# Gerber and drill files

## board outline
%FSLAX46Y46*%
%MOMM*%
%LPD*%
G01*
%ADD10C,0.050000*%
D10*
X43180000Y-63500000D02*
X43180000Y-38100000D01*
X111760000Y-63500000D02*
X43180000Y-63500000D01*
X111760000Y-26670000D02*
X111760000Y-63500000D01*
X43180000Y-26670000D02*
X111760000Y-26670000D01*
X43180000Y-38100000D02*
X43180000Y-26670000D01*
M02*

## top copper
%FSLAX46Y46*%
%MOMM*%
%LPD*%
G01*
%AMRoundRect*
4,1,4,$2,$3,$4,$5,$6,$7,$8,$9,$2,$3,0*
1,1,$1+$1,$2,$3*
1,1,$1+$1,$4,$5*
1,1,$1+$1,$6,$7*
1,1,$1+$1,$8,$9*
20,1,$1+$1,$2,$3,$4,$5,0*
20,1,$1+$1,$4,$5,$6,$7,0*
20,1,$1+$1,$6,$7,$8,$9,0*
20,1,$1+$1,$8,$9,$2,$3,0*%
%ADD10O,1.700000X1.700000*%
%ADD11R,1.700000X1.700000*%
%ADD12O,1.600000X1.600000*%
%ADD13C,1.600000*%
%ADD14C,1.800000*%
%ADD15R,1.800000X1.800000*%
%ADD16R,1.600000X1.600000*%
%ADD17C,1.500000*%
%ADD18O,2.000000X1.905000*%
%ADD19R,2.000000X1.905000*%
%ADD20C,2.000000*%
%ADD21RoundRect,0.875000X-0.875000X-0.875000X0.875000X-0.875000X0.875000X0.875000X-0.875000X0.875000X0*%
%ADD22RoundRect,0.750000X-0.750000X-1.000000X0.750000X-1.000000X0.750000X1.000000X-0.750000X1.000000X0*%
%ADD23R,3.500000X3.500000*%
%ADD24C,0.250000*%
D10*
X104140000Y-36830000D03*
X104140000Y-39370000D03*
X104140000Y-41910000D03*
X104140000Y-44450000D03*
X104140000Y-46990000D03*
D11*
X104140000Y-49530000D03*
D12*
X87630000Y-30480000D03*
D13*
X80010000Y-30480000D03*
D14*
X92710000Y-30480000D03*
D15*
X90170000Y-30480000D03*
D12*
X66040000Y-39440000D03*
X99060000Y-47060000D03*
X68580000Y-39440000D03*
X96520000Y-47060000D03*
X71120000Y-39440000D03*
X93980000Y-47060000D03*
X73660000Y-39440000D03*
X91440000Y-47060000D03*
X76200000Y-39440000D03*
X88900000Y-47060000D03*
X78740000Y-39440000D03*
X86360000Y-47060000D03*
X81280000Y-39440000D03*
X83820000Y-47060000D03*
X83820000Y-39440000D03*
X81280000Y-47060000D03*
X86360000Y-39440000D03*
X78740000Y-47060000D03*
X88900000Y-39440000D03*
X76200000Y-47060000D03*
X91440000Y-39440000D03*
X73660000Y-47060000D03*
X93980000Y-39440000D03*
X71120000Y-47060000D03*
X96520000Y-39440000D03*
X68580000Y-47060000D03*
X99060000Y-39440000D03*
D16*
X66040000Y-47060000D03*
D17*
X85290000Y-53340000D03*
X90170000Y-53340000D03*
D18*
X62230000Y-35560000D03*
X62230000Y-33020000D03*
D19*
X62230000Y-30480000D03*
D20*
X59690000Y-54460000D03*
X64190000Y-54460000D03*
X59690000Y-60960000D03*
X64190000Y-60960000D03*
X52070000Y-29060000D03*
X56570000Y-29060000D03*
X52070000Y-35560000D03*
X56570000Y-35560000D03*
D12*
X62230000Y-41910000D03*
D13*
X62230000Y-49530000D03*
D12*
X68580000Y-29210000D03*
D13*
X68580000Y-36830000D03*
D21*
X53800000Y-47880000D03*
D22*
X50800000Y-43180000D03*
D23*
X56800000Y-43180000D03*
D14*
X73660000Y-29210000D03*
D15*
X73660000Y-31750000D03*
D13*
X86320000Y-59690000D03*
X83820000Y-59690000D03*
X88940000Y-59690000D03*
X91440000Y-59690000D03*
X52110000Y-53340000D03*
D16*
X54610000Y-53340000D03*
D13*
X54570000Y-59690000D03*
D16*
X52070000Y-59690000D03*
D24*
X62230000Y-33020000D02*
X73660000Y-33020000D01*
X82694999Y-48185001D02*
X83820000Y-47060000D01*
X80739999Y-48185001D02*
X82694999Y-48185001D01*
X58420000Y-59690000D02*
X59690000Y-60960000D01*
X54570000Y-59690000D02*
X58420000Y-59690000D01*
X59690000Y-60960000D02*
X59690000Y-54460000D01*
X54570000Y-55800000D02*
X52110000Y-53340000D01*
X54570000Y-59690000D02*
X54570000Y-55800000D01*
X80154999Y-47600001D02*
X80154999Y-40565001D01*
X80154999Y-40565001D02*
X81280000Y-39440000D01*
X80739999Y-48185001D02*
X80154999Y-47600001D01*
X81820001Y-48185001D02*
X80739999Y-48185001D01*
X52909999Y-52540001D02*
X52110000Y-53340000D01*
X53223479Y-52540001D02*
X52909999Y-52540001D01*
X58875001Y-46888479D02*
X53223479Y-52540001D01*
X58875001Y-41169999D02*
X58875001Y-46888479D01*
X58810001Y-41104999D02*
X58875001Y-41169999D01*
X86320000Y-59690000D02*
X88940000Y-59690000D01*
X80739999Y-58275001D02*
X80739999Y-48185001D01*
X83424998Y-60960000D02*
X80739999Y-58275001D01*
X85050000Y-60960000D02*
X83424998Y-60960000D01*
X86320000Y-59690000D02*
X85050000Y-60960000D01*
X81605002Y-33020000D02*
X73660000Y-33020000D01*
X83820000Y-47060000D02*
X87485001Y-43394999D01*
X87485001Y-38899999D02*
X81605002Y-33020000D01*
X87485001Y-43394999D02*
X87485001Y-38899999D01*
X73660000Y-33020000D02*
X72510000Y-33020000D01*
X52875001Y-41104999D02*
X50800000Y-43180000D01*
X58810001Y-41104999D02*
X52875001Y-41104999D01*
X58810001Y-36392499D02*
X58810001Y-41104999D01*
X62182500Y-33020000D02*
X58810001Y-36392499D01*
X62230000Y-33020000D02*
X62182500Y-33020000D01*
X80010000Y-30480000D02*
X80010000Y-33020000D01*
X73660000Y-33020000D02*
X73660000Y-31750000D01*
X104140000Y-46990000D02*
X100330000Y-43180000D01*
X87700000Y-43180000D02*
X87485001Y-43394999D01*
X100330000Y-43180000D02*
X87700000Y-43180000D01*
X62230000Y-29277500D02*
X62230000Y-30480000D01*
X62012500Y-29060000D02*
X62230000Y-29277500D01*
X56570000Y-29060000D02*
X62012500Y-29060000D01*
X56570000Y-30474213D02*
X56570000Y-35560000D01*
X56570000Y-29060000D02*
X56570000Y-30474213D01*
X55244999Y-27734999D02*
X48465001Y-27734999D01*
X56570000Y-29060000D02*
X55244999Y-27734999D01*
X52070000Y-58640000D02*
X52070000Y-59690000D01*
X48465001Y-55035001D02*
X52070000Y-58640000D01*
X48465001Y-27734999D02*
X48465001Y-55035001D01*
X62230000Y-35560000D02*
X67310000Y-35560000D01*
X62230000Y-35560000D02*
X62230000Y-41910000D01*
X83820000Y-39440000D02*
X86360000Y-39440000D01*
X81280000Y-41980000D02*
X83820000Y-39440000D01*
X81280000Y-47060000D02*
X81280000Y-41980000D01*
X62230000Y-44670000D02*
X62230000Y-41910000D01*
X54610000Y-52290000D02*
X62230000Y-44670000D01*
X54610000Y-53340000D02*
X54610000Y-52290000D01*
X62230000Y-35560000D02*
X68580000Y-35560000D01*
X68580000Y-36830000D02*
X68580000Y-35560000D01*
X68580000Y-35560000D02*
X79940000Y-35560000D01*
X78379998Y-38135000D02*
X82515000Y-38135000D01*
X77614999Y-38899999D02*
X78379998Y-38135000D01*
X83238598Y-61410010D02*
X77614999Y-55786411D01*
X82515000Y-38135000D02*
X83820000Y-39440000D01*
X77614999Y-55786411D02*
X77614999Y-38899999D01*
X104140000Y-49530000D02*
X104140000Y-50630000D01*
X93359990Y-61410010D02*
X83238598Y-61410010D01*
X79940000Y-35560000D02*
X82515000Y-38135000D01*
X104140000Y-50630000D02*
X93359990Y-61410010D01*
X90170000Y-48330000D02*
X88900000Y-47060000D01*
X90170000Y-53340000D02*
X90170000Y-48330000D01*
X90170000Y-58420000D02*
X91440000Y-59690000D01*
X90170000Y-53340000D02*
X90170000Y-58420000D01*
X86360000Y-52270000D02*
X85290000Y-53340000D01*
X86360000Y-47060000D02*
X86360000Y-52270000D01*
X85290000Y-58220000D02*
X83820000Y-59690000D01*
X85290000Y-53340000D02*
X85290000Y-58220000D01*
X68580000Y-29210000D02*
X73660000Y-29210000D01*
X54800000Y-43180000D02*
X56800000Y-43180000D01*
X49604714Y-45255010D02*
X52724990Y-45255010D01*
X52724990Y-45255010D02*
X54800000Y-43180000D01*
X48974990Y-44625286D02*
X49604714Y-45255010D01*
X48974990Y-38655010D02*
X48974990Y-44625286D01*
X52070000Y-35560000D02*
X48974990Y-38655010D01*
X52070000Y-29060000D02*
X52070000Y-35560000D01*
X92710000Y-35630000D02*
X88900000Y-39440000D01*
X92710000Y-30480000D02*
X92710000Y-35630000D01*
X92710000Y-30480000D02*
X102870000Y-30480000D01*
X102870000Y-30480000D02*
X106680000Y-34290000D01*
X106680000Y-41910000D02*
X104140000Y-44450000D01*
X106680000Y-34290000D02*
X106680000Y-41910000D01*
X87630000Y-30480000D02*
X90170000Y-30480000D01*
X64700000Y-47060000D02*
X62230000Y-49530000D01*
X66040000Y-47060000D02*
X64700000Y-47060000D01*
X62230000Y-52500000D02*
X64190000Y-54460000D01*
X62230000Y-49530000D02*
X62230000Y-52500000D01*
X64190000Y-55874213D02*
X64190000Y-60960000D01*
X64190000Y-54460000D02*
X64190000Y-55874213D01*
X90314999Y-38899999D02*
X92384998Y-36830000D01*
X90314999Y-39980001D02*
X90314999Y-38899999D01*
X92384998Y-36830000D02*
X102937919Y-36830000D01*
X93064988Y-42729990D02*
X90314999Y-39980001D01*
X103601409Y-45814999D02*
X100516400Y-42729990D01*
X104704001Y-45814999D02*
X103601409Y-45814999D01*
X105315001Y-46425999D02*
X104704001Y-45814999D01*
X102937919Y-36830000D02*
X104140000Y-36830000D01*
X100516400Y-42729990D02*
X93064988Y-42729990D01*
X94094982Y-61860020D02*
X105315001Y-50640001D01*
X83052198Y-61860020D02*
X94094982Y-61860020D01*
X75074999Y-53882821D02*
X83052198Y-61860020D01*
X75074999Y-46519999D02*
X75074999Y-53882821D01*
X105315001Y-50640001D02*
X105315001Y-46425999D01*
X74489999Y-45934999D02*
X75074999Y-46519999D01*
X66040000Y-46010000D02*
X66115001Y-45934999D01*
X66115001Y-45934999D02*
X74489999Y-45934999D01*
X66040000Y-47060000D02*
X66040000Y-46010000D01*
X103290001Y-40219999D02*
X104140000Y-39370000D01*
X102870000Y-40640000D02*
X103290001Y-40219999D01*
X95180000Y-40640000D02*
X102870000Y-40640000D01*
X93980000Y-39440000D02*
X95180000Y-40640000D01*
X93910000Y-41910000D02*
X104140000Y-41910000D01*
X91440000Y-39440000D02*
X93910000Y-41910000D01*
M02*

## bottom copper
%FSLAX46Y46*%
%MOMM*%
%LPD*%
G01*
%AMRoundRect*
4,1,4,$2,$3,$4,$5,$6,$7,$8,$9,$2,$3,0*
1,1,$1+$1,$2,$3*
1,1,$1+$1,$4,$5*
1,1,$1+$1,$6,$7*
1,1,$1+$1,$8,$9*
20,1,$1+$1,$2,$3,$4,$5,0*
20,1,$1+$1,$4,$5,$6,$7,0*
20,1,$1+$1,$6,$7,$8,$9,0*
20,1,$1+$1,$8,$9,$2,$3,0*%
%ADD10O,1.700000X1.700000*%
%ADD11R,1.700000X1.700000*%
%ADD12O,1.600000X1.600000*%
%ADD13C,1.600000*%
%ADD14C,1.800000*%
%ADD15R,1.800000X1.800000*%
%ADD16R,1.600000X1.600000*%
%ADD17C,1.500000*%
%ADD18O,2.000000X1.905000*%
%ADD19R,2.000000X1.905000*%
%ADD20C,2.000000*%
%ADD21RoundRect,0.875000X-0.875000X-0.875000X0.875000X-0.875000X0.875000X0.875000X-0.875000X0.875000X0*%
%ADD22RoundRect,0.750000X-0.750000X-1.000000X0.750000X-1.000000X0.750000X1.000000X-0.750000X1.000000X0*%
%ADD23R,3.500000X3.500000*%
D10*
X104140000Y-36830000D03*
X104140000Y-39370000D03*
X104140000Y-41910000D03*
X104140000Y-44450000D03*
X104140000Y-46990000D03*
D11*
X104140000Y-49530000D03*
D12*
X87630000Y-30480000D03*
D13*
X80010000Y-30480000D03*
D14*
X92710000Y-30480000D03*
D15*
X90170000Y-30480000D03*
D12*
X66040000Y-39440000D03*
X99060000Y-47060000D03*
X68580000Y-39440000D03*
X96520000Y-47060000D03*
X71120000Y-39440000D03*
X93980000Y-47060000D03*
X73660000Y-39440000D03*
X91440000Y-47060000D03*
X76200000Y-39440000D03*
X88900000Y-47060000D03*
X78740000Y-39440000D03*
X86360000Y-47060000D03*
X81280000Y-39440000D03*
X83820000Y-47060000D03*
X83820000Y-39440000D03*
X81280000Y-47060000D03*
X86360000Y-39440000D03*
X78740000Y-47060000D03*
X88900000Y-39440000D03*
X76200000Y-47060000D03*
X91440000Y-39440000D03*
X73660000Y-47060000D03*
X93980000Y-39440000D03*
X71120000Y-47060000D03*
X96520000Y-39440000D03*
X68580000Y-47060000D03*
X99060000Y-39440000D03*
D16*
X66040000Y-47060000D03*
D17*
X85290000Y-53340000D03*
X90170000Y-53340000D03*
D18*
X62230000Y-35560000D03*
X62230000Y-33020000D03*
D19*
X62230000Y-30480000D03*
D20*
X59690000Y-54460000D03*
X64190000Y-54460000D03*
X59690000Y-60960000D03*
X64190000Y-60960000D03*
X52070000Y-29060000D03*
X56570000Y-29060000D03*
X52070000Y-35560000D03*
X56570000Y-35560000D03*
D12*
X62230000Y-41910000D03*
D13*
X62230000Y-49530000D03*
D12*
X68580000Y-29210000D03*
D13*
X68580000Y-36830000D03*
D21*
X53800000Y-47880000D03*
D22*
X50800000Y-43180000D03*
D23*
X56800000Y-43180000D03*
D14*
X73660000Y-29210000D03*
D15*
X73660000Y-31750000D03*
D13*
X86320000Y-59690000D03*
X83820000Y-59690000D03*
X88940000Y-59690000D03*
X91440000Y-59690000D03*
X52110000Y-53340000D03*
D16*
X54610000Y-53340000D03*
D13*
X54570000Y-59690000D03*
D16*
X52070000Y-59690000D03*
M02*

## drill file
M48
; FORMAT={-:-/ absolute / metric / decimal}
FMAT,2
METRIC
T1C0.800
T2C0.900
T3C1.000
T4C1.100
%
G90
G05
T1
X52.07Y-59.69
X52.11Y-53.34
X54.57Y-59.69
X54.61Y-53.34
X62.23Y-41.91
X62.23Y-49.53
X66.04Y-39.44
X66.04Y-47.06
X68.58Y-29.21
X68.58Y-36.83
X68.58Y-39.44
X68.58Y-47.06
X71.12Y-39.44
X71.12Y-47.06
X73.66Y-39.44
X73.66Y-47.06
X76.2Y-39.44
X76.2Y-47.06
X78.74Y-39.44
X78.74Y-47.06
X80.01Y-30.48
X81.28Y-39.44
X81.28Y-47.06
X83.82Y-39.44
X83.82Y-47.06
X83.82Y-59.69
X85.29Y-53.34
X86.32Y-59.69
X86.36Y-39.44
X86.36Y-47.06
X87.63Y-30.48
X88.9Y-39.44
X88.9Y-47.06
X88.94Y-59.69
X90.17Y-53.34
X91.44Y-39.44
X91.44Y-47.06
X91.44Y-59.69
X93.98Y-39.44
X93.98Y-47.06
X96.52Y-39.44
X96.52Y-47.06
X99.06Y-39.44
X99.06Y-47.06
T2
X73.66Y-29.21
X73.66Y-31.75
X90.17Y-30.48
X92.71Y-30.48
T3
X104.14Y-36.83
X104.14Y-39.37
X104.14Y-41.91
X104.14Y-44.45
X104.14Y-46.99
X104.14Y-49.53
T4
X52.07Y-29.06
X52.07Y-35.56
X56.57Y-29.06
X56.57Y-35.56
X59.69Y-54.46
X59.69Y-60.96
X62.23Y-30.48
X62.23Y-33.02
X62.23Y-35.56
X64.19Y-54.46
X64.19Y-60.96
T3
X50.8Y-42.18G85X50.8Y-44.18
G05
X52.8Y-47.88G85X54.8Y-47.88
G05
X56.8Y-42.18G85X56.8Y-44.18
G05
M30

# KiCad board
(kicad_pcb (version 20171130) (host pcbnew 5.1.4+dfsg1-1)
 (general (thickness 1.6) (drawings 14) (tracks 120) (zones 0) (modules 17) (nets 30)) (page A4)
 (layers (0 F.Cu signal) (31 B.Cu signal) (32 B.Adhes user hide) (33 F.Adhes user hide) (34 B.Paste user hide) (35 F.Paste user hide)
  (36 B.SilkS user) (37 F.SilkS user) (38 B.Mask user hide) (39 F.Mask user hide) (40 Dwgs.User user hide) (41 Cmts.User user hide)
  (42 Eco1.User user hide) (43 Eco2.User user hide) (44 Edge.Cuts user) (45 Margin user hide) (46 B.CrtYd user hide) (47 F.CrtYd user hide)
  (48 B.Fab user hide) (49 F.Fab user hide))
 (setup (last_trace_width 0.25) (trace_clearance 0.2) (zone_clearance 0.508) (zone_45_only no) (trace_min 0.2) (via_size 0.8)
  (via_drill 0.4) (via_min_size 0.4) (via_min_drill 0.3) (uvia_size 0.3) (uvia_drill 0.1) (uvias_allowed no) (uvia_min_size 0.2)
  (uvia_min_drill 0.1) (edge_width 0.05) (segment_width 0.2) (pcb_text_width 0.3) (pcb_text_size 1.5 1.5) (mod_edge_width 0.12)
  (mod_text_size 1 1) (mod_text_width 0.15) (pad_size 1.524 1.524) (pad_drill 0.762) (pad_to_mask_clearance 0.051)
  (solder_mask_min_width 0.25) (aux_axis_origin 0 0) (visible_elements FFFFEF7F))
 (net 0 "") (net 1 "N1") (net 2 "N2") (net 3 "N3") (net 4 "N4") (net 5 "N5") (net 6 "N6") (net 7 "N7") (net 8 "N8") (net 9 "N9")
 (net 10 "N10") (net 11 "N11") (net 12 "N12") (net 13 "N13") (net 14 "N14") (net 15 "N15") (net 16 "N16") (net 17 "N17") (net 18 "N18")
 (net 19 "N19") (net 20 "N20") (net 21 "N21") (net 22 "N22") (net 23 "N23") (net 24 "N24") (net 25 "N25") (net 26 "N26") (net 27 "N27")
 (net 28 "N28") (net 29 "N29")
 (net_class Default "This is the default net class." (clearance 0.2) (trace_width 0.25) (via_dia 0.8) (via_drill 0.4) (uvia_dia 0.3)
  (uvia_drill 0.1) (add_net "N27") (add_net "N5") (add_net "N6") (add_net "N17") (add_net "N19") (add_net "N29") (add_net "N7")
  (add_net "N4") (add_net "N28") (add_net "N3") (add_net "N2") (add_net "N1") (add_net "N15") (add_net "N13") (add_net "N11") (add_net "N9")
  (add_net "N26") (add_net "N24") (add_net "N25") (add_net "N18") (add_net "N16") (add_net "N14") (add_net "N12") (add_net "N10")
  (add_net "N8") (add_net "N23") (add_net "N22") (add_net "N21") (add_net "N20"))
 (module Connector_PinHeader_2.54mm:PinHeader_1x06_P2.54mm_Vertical (layer F.Cu) (at 104.14 49.53 180)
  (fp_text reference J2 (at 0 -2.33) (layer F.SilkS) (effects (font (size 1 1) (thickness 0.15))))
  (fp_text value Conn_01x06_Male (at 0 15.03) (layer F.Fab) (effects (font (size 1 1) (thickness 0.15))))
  (pad 6 thru_hole oval (at 0 12.7 180) (size 1.7 1.7) (drill 1) (layers *.Cu *.Mask) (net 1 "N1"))
  (pad 5 thru_hole oval (at 0 10.16 180) (size 1.7 1.7) (drill 1) (layers *.Cu *.Mask) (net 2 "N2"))
  (pad 4 thru_hole oval (at 0 7.62 180) (size 1.7 1.7) (drill 1) (layers *.Cu *.Mask) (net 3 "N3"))
  (pad 3 thru_hole oval (at 0 5.08 180) (size 1.7 1.7) (drill 1) (layers *.Cu *.Mask) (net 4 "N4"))
  (pad 2 thru_hole oval (at 0 2.54 180) (size 1.7 1.7) (drill 1) (layers *.Cu *.Mask) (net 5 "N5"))
  (pad 1 thru_hole rect (at 0 0 180) (size 1.7 1.7) (drill 1) (layers *.Cu *.Mask) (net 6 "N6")))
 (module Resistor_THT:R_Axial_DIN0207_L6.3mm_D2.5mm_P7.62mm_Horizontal (layer F.Cu) (at 80.01 30.48)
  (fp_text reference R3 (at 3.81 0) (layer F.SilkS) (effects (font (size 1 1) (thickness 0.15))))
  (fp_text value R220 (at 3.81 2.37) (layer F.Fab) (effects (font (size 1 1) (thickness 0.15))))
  (pad 2 thru_hole oval (at 7.62 0) (size 1.6 1.6) (drill 0.8) (layers *.Cu *.Mask) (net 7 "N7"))
  (pad 1 thru_hole circle (at 0 0) (size 1.6 1.6) (drill 0.8) (layers *.Cu *.Mask) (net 5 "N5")))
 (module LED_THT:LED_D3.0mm (layer F.Cu) (at 90.17 30.48)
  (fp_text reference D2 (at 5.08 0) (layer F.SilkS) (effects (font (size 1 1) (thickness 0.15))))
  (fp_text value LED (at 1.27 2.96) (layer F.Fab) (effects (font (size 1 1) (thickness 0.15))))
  (pad 2 thru_hole circle (at 2.54 0) (size 1.8 1.8) (drill 0.9) (layers *.Cu *.Mask) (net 4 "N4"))
  (pad 1 thru_hole rect (at 0 0) (size 1.8 1.8) (drill 0.9) (layers *.Cu *.Mask) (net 7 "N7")))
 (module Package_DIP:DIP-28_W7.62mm (layer F.Cu) (at 66.04 47.06 90)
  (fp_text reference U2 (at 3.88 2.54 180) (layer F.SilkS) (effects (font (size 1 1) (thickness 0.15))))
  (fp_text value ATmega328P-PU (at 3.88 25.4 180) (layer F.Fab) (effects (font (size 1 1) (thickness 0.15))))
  (pad 28 thru_hole oval (at 7.62 0 90) (size 1.6 1.6) (drill 0.8) (layers *.Cu *.Mask) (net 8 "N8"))
  (pad 14 thru_hole oval (at 0 33.02 90) (size 1.6 1.6) (drill 0.8) (layers *.Cu *.Mask) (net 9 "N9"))
  (pad 27 thru_hole oval (at 7.62 2.54 90) (size 1.6 1.6) (drill 0.8) (layers *.Cu *.Mask) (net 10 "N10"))
  (pad 13 thru_hole oval (at 0 30.48 90) (size 1.6 1.6) (drill 0.8) (layers *.Cu *.Mask) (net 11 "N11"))
  (pad 26 thru_hole oval (at 7.62 5.08 90) (size 1.6 1.6) (drill 0.8) (layers *.Cu *.Mask) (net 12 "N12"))
  (pad 12 thru_hole oval (at 0 27.94 90) (size 1.6 1.6) (drill 0.8) (layers *.Cu *.Mask) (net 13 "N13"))
  (pad 25 thru_hole oval (at 7.62 7.62 90) (size 1.6 1.6) (drill 0.8) (layers *.Cu *.Mask) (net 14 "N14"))
  (pad 11 thru_hole oval (at 0 25.4 90) (size 1.6 1.6) (drill 0.8) (layers *.Cu *.Mask) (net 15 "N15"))
  (pad 24 thru_hole oval (at 7.62 10.16 90) (size 1.6 1.6) (drill 0.8) (layers *.Cu *.Mask) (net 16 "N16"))
  (pad 10 thru_hole oval (at 0 22.86 90) (size 1.6 1.6) (drill 0.8) (layers *.Cu *.Mask) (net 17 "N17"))
  (pad 23 thru_hole oval (at 7.62 12.7 90) (size 1.6 1.6) (drill 0.8) (layers *.Cu *.Mask) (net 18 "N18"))
  (pad 9 thru_hole oval (at 0 20.32 90) (size 1.6 1.6) (drill 0.8) (layers *.Cu *.Mask) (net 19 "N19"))
  (pad 22 thru_hole oval (at 7.62 15.24 90) (size 1.6 1.6) (drill 0.8) (layers *.Cu *.Mask) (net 5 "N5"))
  (pad 8 thru_hole oval (at 0 17.78 90) (size 1.6 1.6) (drill 0.8) (layers *.Cu *.Mask) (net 5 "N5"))
  (pad 21 thru_hole oval (at 7.62 17.78 90) (size 1.6 1.6) (drill 0.8) (layers *.Cu *.Mask) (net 6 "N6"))
  (pad 7 thru_hole oval (at 0 15.24 90) (size 1.6 1.6) (drill 0.8) (layers *.Cu *.Mask) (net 6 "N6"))
  (pad 20 thru_hole oval (at 7.62 20.32 90) (size 1.6 1.6) (drill 0.8) (layers *.Cu *.Mask) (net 6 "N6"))
  (pad 6 thru_hole oval (at 0 12.7 90) (size 1.6 1.6) (drill 0.8) (layers *.Cu *.Mask) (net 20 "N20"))
  (pad 19 thru_hole oval (at 7.62 22.86 90) (size 1.6 1.6) (drill 0.8) (layers *.Cu *.Mask) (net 4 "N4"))
  (pad 5 thru_hole oval (at 0 10.16 90) (size 1.6 1.6) (drill 0.8) (layers *.Cu *.Mask) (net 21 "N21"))
  (pad 18 thru_hole oval (at 7.62 25.4 90) (size 1.6 1.6) (drill 0.8) (layers *.Cu *.Mask) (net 3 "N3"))
  (pad 4 thru_hole oval (at 0 7.62 90) (size 1.6 1.6) (drill 0.8) (layers *.Cu *.Mask) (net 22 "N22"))
  (pad 17 thru_hole oval (at 7.62 27.94 90) (size 1.6 1.6) (drill 0.8) (layers *.Cu *.Mask) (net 2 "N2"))
  (pad 3 thru_hole oval (at 0 5.08 90) (size 1.6 1.6) (drill 0.8) (layers *.Cu *.Mask) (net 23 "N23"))
  (pad 16 thru_hole oval (at 7.62 30.48 90) (size 1.6 1.6) (drill 0.8) (layers *.Cu *.Mask) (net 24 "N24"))
  (pad 2 thru_hole oval (at 0 2.54 90) (size 1.6 1.6) (drill 0.8) (layers *.Cu *.Mask) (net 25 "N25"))
  (pad 15 thru_hole oval (at 7.62 33.02 90) (size 1.6 1.6) (drill 0.8) (layers *.Cu *.Mask) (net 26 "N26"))
  (pad 1 thru_hole rect (at 0 0 90) (size 1.6 1.6) (drill 0.8) (layers *.Cu *.Mask) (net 1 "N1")))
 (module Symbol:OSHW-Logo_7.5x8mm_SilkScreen (layer F.Cu) (at 73.66 55.88)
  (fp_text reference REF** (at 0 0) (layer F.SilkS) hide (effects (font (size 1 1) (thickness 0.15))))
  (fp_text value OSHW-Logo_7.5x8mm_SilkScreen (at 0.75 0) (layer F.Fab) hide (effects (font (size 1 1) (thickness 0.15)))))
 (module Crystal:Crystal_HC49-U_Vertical (layer F.Cu) (at 90.17 53.34 180)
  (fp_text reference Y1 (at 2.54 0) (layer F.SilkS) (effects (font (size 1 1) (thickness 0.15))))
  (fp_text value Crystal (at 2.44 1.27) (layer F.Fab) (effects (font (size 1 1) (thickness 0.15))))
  (pad 2 thru_hole circle (at 4.88 0 180) (size 1.5 1.5) (drill 0.8) (layers *.Cu *.Mask) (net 19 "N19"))
  (pad 1 thru_hole circle (at 0 0 180) (size 1.5 1.5) (drill 0.8) (layers *.Cu *.Mask) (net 17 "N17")))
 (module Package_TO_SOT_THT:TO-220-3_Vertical (layer F.Cu) (at 62.23 30.48 270)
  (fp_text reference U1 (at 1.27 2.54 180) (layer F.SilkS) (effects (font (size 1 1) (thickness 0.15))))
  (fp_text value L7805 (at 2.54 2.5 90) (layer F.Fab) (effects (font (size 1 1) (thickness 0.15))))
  (pad 3 thru_hole oval (at 5.08 0 270) (size 1.905 2) (drill 1.1) (layers *.Cu *.Mask) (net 6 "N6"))
  (pad 2 thru_hole oval (at 2.54 0 270) (size 1.905 2) (drill 1.1) (layers *.Cu *.Mask) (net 5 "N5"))
  (pad 1 thru_hole rect (at 0 0 270) (size 1.905 2) (drill 1.1) (layers *.Cu *.Mask) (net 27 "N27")))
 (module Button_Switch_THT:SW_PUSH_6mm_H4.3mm (layer F.Cu) (at 59.69 60.96 90)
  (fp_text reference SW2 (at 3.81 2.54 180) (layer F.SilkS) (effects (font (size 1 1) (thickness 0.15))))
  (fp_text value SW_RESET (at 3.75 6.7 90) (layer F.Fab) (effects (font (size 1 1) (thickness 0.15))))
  (pad 1 thru_hole circle (at 6.5 0 180) (size 2 2) (drill 1.1) (layers *.Cu *.Mask) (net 5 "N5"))
  (pad 2 thru_hole circle (at 6.5 4.5 180) (size 2 2) (drill 1.1) (layers *.Cu *.Mask) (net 1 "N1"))
  (pad 1 thru_hole circle (at 0 0 180) (size 2 2) (drill 1.1) (layers *.Cu *.Mask) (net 5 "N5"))
  (pad 2 thru_hole circle (at 0 4.5 180) (size 2 2) (drill 1.1) (layers *.Cu *.Mask) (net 1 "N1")))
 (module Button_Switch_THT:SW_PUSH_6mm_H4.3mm (layer F.Cu) (at 52.07 35.56 90)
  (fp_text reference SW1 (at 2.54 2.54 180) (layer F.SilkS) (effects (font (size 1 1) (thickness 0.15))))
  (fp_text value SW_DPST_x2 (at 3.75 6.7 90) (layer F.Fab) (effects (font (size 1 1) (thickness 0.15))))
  (pad 1 thru_hole circle (at 6.5 0 180) (size 2 2) (drill 1.1) (layers *.Cu *.Mask) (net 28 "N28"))
  (pad 2 thru_hole circle (at 6.5 4.5 180) (size 2 2) (drill 1.1) (layers *.Cu *.Mask) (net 27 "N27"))
  (pad 1 thru_hole circle (at 0 0 180) (size 2 2) (drill 1.1) (layers *.Cu *.Mask) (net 28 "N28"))
  (pad 2 thru_hole circle (at 0 4.5 180) (size 2 2) (drill 1.1) (layers *.Cu *.Mask) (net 27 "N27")))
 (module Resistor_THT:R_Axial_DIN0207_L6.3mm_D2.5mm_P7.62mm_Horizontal (layer F.Cu) (at 62.23 49.53 90)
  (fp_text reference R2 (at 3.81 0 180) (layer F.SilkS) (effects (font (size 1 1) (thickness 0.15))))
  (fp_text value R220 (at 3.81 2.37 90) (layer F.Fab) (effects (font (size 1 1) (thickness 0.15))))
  (pad 2 thru_hole oval (at 7.62 0 90) (size 1.6 1.6) (drill 0.8) (layers *.Cu *.Mask) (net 6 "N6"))
  (pad 1 thru_hole circle (at 0 0 90) (size 1.6 1.6) (drill 0.8) (layers *.Cu *.Mask) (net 1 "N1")))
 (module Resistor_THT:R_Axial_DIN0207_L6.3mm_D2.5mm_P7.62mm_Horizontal (layer F.Cu) (at 68.58 36.83 90)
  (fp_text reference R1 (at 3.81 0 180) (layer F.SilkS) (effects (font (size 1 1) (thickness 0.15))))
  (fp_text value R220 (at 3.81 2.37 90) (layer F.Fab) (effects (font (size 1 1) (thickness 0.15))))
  (pad 2 thru_hole oval (at 7.62 0 90) (size 1.6 1.6) (drill 0.8) (layers *.Cu *.Mask) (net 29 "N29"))
  (pad 1 thru_hole circle (at 0 0 90) (size 1.6 1.6) (drill 0.8) (layers *.Cu *.Mask) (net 6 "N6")))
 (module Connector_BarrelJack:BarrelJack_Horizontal (layer F.Cu) (at 56.8 43.18)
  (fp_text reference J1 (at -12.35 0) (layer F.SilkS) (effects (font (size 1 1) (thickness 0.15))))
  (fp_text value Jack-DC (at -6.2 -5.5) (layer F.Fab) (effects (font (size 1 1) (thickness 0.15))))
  (pad 3 thru_hole roundrect (at -3 4.7) (size 3.5 3.5) (drill oval 3 1) (layers *.Cu *.Mask) (roundrect_rratio 0.25))
  (pad 2 thru_hole roundrect (at -6 0) (size 3 3.5) (drill oval 1 3) (layers *.Cu *.Mask) (roundrect_rratio 0.25) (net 5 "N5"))
  (pad 1 thru_hole rect (at 0 0) (size 3.5 3.5) (drill oval 1 3) (layers *.Cu *.Mask) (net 28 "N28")))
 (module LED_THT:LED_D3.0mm (layer F.Cu) (at 73.66 31.75 90)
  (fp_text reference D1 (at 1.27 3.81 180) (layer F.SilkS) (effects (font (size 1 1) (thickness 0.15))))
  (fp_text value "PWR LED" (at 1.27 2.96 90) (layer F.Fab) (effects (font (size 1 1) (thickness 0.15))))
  (pad 2 thru_hole circle (at 2.54 0 90) (size 1.8 1.8) (drill 0.9) (layers *.Cu *.Mask) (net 29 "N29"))
  (pad 1 thru_hole rect (at 0 0 90) (size 1.8 1.8) (drill 0.9) (layers *.Cu *.Mask) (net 5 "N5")))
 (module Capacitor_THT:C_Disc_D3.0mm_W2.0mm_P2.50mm (layer F.Cu) (at 83.82 59.69)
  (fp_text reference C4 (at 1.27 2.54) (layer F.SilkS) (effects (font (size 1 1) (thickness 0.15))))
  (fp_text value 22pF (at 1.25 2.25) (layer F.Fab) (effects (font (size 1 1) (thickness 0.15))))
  (pad 2 thru_hole circle (at 2.5 0) (size 1.6 1.6) (drill 0.8) (layers *.Cu *.Mask) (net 5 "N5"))
  (pad 1 thru_hole circle (at 0 0) (size 1.6 1.6) (drill 0.8) (layers *.Cu *.Mask) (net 19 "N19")))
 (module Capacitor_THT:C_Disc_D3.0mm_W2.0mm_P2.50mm (layer F.Cu) (at 91.44 59.69 180)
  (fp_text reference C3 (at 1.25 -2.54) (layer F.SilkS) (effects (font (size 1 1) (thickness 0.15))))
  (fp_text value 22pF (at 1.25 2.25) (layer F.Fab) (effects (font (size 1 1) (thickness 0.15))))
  (pad 2 thru_hole circle (at 2.5 0 180) (size 1.6 1.6) (drill 0.8) (layers *.Cu *.Mask) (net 5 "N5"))
  (pad 1 thru_hole circle (at 0 0 180) (size 1.6 1.6) (drill 0.8) (layers *.Cu *.Mask) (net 17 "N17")))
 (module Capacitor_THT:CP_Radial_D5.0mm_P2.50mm (layer F.Cu) (at 54.61 53.34 180)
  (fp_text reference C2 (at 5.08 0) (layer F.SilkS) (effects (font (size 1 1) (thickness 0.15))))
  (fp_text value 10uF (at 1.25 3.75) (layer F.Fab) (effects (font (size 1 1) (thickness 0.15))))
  (pad 2 thru_hole circle (at 2.5 0 180) (size 1.6 1.6) (drill 0.8) (layers *.Cu *.Mask) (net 5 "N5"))
  (pad 1 thru_hole rect (at 0 0 180) (size 1.6 1.6) (drill 0.8) (layers *.Cu *.Mask) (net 6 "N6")))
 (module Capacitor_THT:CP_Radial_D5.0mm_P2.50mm (layer F.Cu) (at 52.07 59.69)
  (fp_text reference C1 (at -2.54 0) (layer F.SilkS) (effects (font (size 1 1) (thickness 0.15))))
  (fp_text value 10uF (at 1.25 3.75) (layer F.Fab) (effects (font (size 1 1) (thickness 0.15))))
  (pad 2 thru_hole circle (at 2.5 0) (size 1.6 1.6) (drill 0.8) (layers *.Cu *.Mask) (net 5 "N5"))
  (pad 1 thru_hole rect (at 0 0) (size 1.6 1.6) (drill 0.8) (layers *.Cu *.Mask) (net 27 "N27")))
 (gr_line (start 43.18 63.5) (end 43.18 38.1) (layer Edge.Cuts) (width 0.05))
 (gr_line (start 111.76 63.5) (end 43.18 63.5) (layer Edge.Cuts) (width 0.05))
 (gr_line (start 111.76 26.67) (end 111.76 63.5) (layer Edge.Cuts) (width 0.05))
 (gr_line (start 43.18 26.67) (end 111.76 26.67) (layer Edge.Cuts) (width 0.05))
 (gr_line (start 43.18 38.1) (end 43.18 26.67) (layer Edge.Cuts) (width 0.05))
 (segment (start 62.23 33.02) (end 73.66 33.02) (width 0.25) (layer F.Cu) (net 5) (status 30))
 (segment (start 82.694999 48.185001) (end 83.82 47.06) (width 0.25) (layer F.Cu) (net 5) (status 20))
 (segment (start 80.739999 48.185001) (end 82.694999 48.185001) (width 0.25) (layer F.Cu) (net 5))
 (segment (start 58.42 59.69) (end 59.69 60.96) (width 0.25) (layer F.Cu) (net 5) (status 20))
 (segment (start 54.57 59.69) (end 58.42 59.69) (width 0.25) (layer F.Cu) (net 5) (status 10))
 (segment (start 59.69 60.96) (end 59.69 54.46) (width 0.25) (layer F.Cu) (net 5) (status 30))
 (segment (start 54.57 55.8) (end 52.11 53.34) (width 0.25) (layer F.Cu) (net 5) (status 20))
 (segment (start 54.57 59.69) (end 54.57 55.8) (width 0.25) (layer F.Cu) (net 5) (status 10))
 (segment (start 80.154999 47.600001) (end 80.154999 40.565001) (width 0.25) (layer F.Cu) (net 5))
 (segment (start 80.154999 40.565001) (end 81.28 39.44) (width 0.25) (layer F.Cu) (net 5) (status 20))
 (segment (start 80.739999 48.185001) (end 80.154999 47.600001) (width 0.25) (layer F.Cu) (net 5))
 (segment (start 81.820001 48.185001) (end 80.739999 48.185001) (width 0.25) (layer F.Cu) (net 5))
 (segment (start 52.909999 52.540001) (end 52.11 53.34) (width 0.25) (layer F.Cu) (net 5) (status 20))
 (segment (start 53.223479 52.540001) (end 52.909999 52.540001) (width 0.25) (layer F.Cu) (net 5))
 (segment (start 58.875001 46.888479) (end 53.223479 52.540001) (width 0.25) (layer F.Cu) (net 5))
 (segment (start 58.875001 41.169999) (end 58.875001 46.888479) (width 0.25) (layer F.Cu) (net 5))
 (segment (start 58.810001 41.104999) (end 58.875001 41.169999) (width 0.25) (layer F.Cu) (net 5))
 (segment (start 86.32 59.69) (end 88.94 59.69) (width 0.25) (layer F.Cu) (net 5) (status 30))
 (segment (start 80.739999 58.275001) (end 80.739999 48.185001) (width 0.25) (layer F.Cu) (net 5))
 (segment (start 83.424998 60.96) (end 80.739999 58.275001) (width 0.25) (layer F.Cu) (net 5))
 (segment (start 85.05 60.96) (end 83.424998 60.96) (width 0.25) (layer F.Cu) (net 5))
 (segment (start 86.32 59.69) (end 85.05 60.96) (width 0.25) (layer F.Cu) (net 5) (status 10))
 (segment (start 81.605002 33.02) (end 73.66 33.02) (width 0.25) (layer F.Cu) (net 5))
 (segment (start 83.82 47.06) (end 87.485001 43.394999) (width 0.25) (layer F.Cu) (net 5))
 (segment (start 87.485001 38.899999) (end 81.605002 33.02) (width 0.25) (layer F.Cu) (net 5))
 (segment (start 87.485001 43.394999) (end 87.485001 38.899999) (width 0.25) (layer F.Cu) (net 5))
 (segment (start 73.66 33.02) (end 72.51 33.02) (width 0.25) (layer F.Cu) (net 5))
 (segment (start 52.875001 41.104999) (end 50.8 43.18) (width 0.25) (layer F.Cu) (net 5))
 (segment (start 58.810001 41.104999) (end 52.875001 41.104999) (width 0.25) (layer F.Cu) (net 5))
 (segment (start 58.810001 36.392499) (end 58.810001 41.104999) (width 0.25) (layer F.Cu) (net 5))
 (segment (start 62.1825 33.02) (end 58.810001 36.392499) (width 0.25) (layer F.Cu) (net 5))
 (segment (start 62.23 33.02) (end 62.1825 33.02) (width 0.25) (layer F.Cu) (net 5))
 (segment (start 80.01 30.48) (end 80.01 33.02) (width 0.25) (layer F.Cu) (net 5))
 (segment (start 73.66 33.02) (end 73.66 31.75) (width 0.25) (layer F.Cu) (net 5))
 (segment (start 104.14 46.99) (end 100.33 43.18) (width 0.25) (layer F.Cu) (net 5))
 (segment (start 87.7 43.18) (end 87.485001 43.394999) (width 0.25) (layer F.Cu) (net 5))
 (segment (start 100.33 43.18) (end 87.7 43.18) (width 0.25) (layer F.Cu) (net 5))
 (segment (start 62.23 29.2775) (end 62.23 30.48) (width 0.25) (layer F.Cu) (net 27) (status 20))
 (segment (start 62.0125 29.06) (end 62.23 29.2775) (width 0.25) (layer F.Cu) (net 27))
 (segment (start 56.57 29.06) (end 62.0125 29.06) (width 0.25) (layer F.Cu) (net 27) (status 10))
 (segment (start 56.57 30.474213) (end 56.57 35.56) (width 0.25) (layer F.Cu) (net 27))
 (segment (start 56.57 29.06) (end 56.57 30.474213) (width 0.25) (layer F.Cu) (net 27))
 (segment (start 55.244999 27.734999) (end 48.465001 27.734999) (width 0.25) (layer F.Cu) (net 27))
 (segment (start 56.57 29.06) (end 55.244999 27.734999) (width 0.25) (layer F.Cu) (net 27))
 (segment (start 52.07 58.64) (end 52.07 59.69) (width 0.25) (layer F.Cu) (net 27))
 (segment (start 48.465001 55.035001) (end 52.07 58.64) (width 0.25) (layer F.Cu) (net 27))
 (segment (start 48.465001 27.734999) (end 48.465001 55.035001) (width 0.25) (layer F.Cu) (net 27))
 (segment (start 62.23 35.56) (end 67.31 35.56) (width 0.25) (layer F.Cu) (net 6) (status 10))
 (segment (start 62.23 35.56) (end 62.23 41.91) (width 0.25) (layer F.Cu) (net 6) (status 30))
 (segment (start 83.82 39.44) (end 86.36 39.44) (width 0.25) (layer F.Cu) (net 6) (status 30))
 (segment (start 81.28 41.98) (end 83.82 39.44) (width 0.25) (layer F.Cu) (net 6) (status 20))
 (segment (start 81.28 47.06) (end 81.28 41.98) (width 0.25) (layer F.Cu) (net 6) (status 10))
 (segment (start 62.23 44.67) (end 62.23 41.91) (width 0.25) (layer F.Cu) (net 6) (status 20))
 (segment (start 54.61 52.29) (end 62.23 44.67) (width 0.25) (layer F.Cu) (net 6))
 (segment (start 54.61 53.34) (end 54.61 52.29) (width 0.25) (layer F.Cu) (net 6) (status 10))
 (segment (start 62.23 35.56) (end 68.58 35.56) (width 0.25) (layer F.Cu) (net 6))
 (segment (start 68.58 36.83) (end 68.58 35.56) (width 0.25) (layer F.Cu) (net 6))
 (segment (start 68.58 35.56) (end 79.94 35.56) (width 0.25) (layer F.Cu) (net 6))
 (segment (start 78.379998 38.135) (end 82.515 38.135) (width 0.25) (layer F.Cu) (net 6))
 (segment (start 77.614999 38.899999) (end 78.379998 38.135) (width 0.25) (layer F.Cu) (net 6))
 (segment (start 83.238598 61.41001) (end 77.614999 55.786411) (width 0.25) (layer F.Cu) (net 6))
 (segment (start 82.515 38.135) (end 83.82 39.44) (width 0.25) (layer F.Cu) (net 6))
 (segment (start 77.614999 55.786411) (end 77.614999 38.899999) (width 0.25) (layer F.Cu) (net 6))
 (segment (start 104.14 49.53) (end 104.14 50.63) (width 0.25) (layer F.Cu) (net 6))
 (segment (start 93.35999 61.41001) (end 83.238598 61.41001) (width 0.25) (layer F.Cu) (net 6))
 (segment (start 79.94 35.56) (end 82.515 38.135) (width 0.25) (layer F.Cu) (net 6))
 (segment (start 104.14 50.63) (end 93.35999 61.41001) (width 0.25) (layer F.Cu) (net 6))
 (segment (start 90.17 48.33) (end 88.9 47.06) (width 0.25) (layer F.Cu) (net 17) (status 20))
 (segment (start 90.17 53.34) (end 90.17 48.33) (width 0.25) (layer F.Cu) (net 17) (status 10))
 (segment (start 90.17 58.42) (end 91.44 59.69) (width 0.25) (layer F.Cu) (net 17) (status 20))
 (segment (start 90.17 53.34) (end 90.17 58.42) (width 0.25) (layer F.Cu) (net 17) (status 10))
 (segment (start 86.36 52.27) (end 85.29 53.34) (width 0.25) (layer F.Cu) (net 19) (status 20))
 (segment (start 86.36 47.06) (end 86.36 52.27) (width 0.25) (layer F.Cu) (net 19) (status 10))
 (segment (start 85.29 58.22) (end 83.82 59.69) (width 0.25) (layer F.Cu) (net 19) (status 20))
 (segment (start 85.29 53.34) (end 85.29 58.22) (width 0.25) (layer F.Cu) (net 19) (status 10))
 (segment (start 68.58 29.21) (end 73.66 29.21) (width 0.25) (layer F.Cu) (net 29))
 (segment (start 54.8 43.18) (end 56.8 43.18) (width 0.25) (layer F.Cu) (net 28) (status 20))
 (segment (start 49.604714 45.25501) (end 52.72499 45.25501) (width 0.25) (layer F.Cu) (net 28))
 (segment (start 52.72499 45.25501) (end 54.8 43.18) (width 0.25) (layer F.Cu) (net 28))
 (segment (start 48.97499 44.625286) (end 49.604714 45.25501) (width 0.25) (layer F.Cu) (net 28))
 (segment (start 48.97499 38.65501) (end 48.97499 44.625286) (width 0.25) (layer F.Cu) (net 28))
 (segment (start 52.07 35.56) (end 48.97499 38.65501) (width 0.25) (layer F.Cu) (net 28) (status 10))
 (segment (start 52.07 29.06) (end 52.07 35.56) (width 0.25) (layer F.Cu) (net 28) (status 30))
 (segment (start 92.71 35.63) (end 88.9 39.44) (width 0.25) (layer F.Cu) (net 4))
 (segment (start 92.71 30.48) (end 92.71 35.63) (width 0.25) (layer F.Cu) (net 4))
 (segment (start 92.71 30.48) (end 102.87 30.48) (width 0.25) (layer F.Cu) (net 4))
 (segment (start 102.87 30.48) (end 106.68 34.29) (width 0.25) (layer F.Cu) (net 4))
 (segment (start 106.68 41.91) (end 104.14 44.45) (width 0.25) (layer F.Cu) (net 4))
 (segment (start 106.68 34.29) (end 106.68 41.91) (width 0.25) (layer F.Cu) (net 4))
 (segment (start 87.63 30.48) (end 90.17 30.48) (width 0.25) (layer F.Cu) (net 7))
 (segment (start 64.7 47.06) (end 62.23 49.53) (width 0.25) (layer F.Cu) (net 1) (status 20))
 (segment (start 66.04 47.06) (end 64.7 47.06) (width 0.25) (layer F.Cu) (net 1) (status 10))
 (segment (start 62.23 52.5) (end 64.19 54.46) (width 0.25) (layer F.Cu) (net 1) (status 20))
 (segment (start 62.23 49.53) (end 62.23 52.5) (width 0.25) (layer F.Cu) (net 1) (status 10))
 (segment (start 64.19 55.874213) (end 64.19 60.96) (width 0.25) (layer F.Cu) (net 1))
 (segment (start 64.19 54.46) (end 64.19 55.874213) (width 0.25) (layer F.Cu) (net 1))
 (segment (start 90.314999 38.899999) (end 92.384998 36.83) (width 0.25) (layer F.Cu) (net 1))
 (segment (start 90.314999 39.980001) (end 90.314999 38.899999) (width 0.25) (layer F.Cu) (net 1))
 (segment (start 92.384998 36.83) (end 102.937919 36.83) (width 0.25) (layer F.Cu) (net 1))
 (segment (start 93.064988 42.72999) (end 90.314999 39.980001) (width 0.25) (layer F.Cu) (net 1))
 (segment (start 103.601409 45.814999) (end 100.5164 42.72999) (width 0.25) (layer F.Cu) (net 1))
 (segment (start 104.704001 45.814999) (end 103.601409 45.814999) (width 0.25) (layer F.Cu) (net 1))
 (segment (start 105.315001 46.425999) (end 104.704001 45.814999) (width 0.25) (layer F.Cu) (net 1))
 (segment (start 102.937919 36.83) (end 104.14 36.83) (width 0.25) (layer F.Cu) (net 1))
 (segment (start 100.5164 42.72999) (end 93.064988 42.72999) (width 0.25) (layer F.Cu) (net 1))
 (segment (start 94.094982 61.86002) (end 105.315001 50.640001) (width 0.25) (layer F.Cu) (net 1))
 (segment (start 83.052198 61.86002) (end 94.094982 61.86002) (width 0.25) (layer F.Cu) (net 1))
 (segment (start 75.074999 53.882821) (end 83.052198 61.86002) (width 0.25) (layer F.Cu) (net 1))
 (segment (start 75.074999 46.519999) (end 75.074999 53.882821) (width 0.25) (layer F.Cu) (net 1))
 (segment (start 105.315001 50.640001) (end 105.315001 46.425999) (width 0.25) (layer F.Cu) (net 1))
 (segment (start 74.489999 45.934999) (end 75.074999 46.519999) (width 0.25) (layer F.Cu) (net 1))
 (segment (start 66.04 46.01) (end 66.115001 45.934999) (width 0.25) (layer F.Cu) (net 1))
 (segment (start 66.115001 45.934999) (end 74.489999 45.934999) (width 0.25) (layer F.Cu) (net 1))
 (segment (start 66.04 47.06) (end 66.04 46.01) (width 0.25) (layer F.Cu) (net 1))
 (segment (start 103.290001 40.219999) (end 104.14 39.37) (width 0.25) (layer F.Cu) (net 2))
 (segment (start 102.87 40.64) (end 103.290001 40.219999) (width 0.25) (layer F.Cu) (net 2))
 (segment (start 95.18 40.64) (end 102.87 40.64) (width 0.25) (layer F.Cu) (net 2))
 (segment (start 93.98 39.44) (end 95.18 40.64) (width 0.25) (layer F.Cu) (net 2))
 (segment (start 93.91 41.91) (end 104.14 41.91) (width 0.25) (layer F.Cu) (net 3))
 (segment (start 91.44 39.44) (end 93.91 41.91) (width 0.25) (layer F.Cu) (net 3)))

